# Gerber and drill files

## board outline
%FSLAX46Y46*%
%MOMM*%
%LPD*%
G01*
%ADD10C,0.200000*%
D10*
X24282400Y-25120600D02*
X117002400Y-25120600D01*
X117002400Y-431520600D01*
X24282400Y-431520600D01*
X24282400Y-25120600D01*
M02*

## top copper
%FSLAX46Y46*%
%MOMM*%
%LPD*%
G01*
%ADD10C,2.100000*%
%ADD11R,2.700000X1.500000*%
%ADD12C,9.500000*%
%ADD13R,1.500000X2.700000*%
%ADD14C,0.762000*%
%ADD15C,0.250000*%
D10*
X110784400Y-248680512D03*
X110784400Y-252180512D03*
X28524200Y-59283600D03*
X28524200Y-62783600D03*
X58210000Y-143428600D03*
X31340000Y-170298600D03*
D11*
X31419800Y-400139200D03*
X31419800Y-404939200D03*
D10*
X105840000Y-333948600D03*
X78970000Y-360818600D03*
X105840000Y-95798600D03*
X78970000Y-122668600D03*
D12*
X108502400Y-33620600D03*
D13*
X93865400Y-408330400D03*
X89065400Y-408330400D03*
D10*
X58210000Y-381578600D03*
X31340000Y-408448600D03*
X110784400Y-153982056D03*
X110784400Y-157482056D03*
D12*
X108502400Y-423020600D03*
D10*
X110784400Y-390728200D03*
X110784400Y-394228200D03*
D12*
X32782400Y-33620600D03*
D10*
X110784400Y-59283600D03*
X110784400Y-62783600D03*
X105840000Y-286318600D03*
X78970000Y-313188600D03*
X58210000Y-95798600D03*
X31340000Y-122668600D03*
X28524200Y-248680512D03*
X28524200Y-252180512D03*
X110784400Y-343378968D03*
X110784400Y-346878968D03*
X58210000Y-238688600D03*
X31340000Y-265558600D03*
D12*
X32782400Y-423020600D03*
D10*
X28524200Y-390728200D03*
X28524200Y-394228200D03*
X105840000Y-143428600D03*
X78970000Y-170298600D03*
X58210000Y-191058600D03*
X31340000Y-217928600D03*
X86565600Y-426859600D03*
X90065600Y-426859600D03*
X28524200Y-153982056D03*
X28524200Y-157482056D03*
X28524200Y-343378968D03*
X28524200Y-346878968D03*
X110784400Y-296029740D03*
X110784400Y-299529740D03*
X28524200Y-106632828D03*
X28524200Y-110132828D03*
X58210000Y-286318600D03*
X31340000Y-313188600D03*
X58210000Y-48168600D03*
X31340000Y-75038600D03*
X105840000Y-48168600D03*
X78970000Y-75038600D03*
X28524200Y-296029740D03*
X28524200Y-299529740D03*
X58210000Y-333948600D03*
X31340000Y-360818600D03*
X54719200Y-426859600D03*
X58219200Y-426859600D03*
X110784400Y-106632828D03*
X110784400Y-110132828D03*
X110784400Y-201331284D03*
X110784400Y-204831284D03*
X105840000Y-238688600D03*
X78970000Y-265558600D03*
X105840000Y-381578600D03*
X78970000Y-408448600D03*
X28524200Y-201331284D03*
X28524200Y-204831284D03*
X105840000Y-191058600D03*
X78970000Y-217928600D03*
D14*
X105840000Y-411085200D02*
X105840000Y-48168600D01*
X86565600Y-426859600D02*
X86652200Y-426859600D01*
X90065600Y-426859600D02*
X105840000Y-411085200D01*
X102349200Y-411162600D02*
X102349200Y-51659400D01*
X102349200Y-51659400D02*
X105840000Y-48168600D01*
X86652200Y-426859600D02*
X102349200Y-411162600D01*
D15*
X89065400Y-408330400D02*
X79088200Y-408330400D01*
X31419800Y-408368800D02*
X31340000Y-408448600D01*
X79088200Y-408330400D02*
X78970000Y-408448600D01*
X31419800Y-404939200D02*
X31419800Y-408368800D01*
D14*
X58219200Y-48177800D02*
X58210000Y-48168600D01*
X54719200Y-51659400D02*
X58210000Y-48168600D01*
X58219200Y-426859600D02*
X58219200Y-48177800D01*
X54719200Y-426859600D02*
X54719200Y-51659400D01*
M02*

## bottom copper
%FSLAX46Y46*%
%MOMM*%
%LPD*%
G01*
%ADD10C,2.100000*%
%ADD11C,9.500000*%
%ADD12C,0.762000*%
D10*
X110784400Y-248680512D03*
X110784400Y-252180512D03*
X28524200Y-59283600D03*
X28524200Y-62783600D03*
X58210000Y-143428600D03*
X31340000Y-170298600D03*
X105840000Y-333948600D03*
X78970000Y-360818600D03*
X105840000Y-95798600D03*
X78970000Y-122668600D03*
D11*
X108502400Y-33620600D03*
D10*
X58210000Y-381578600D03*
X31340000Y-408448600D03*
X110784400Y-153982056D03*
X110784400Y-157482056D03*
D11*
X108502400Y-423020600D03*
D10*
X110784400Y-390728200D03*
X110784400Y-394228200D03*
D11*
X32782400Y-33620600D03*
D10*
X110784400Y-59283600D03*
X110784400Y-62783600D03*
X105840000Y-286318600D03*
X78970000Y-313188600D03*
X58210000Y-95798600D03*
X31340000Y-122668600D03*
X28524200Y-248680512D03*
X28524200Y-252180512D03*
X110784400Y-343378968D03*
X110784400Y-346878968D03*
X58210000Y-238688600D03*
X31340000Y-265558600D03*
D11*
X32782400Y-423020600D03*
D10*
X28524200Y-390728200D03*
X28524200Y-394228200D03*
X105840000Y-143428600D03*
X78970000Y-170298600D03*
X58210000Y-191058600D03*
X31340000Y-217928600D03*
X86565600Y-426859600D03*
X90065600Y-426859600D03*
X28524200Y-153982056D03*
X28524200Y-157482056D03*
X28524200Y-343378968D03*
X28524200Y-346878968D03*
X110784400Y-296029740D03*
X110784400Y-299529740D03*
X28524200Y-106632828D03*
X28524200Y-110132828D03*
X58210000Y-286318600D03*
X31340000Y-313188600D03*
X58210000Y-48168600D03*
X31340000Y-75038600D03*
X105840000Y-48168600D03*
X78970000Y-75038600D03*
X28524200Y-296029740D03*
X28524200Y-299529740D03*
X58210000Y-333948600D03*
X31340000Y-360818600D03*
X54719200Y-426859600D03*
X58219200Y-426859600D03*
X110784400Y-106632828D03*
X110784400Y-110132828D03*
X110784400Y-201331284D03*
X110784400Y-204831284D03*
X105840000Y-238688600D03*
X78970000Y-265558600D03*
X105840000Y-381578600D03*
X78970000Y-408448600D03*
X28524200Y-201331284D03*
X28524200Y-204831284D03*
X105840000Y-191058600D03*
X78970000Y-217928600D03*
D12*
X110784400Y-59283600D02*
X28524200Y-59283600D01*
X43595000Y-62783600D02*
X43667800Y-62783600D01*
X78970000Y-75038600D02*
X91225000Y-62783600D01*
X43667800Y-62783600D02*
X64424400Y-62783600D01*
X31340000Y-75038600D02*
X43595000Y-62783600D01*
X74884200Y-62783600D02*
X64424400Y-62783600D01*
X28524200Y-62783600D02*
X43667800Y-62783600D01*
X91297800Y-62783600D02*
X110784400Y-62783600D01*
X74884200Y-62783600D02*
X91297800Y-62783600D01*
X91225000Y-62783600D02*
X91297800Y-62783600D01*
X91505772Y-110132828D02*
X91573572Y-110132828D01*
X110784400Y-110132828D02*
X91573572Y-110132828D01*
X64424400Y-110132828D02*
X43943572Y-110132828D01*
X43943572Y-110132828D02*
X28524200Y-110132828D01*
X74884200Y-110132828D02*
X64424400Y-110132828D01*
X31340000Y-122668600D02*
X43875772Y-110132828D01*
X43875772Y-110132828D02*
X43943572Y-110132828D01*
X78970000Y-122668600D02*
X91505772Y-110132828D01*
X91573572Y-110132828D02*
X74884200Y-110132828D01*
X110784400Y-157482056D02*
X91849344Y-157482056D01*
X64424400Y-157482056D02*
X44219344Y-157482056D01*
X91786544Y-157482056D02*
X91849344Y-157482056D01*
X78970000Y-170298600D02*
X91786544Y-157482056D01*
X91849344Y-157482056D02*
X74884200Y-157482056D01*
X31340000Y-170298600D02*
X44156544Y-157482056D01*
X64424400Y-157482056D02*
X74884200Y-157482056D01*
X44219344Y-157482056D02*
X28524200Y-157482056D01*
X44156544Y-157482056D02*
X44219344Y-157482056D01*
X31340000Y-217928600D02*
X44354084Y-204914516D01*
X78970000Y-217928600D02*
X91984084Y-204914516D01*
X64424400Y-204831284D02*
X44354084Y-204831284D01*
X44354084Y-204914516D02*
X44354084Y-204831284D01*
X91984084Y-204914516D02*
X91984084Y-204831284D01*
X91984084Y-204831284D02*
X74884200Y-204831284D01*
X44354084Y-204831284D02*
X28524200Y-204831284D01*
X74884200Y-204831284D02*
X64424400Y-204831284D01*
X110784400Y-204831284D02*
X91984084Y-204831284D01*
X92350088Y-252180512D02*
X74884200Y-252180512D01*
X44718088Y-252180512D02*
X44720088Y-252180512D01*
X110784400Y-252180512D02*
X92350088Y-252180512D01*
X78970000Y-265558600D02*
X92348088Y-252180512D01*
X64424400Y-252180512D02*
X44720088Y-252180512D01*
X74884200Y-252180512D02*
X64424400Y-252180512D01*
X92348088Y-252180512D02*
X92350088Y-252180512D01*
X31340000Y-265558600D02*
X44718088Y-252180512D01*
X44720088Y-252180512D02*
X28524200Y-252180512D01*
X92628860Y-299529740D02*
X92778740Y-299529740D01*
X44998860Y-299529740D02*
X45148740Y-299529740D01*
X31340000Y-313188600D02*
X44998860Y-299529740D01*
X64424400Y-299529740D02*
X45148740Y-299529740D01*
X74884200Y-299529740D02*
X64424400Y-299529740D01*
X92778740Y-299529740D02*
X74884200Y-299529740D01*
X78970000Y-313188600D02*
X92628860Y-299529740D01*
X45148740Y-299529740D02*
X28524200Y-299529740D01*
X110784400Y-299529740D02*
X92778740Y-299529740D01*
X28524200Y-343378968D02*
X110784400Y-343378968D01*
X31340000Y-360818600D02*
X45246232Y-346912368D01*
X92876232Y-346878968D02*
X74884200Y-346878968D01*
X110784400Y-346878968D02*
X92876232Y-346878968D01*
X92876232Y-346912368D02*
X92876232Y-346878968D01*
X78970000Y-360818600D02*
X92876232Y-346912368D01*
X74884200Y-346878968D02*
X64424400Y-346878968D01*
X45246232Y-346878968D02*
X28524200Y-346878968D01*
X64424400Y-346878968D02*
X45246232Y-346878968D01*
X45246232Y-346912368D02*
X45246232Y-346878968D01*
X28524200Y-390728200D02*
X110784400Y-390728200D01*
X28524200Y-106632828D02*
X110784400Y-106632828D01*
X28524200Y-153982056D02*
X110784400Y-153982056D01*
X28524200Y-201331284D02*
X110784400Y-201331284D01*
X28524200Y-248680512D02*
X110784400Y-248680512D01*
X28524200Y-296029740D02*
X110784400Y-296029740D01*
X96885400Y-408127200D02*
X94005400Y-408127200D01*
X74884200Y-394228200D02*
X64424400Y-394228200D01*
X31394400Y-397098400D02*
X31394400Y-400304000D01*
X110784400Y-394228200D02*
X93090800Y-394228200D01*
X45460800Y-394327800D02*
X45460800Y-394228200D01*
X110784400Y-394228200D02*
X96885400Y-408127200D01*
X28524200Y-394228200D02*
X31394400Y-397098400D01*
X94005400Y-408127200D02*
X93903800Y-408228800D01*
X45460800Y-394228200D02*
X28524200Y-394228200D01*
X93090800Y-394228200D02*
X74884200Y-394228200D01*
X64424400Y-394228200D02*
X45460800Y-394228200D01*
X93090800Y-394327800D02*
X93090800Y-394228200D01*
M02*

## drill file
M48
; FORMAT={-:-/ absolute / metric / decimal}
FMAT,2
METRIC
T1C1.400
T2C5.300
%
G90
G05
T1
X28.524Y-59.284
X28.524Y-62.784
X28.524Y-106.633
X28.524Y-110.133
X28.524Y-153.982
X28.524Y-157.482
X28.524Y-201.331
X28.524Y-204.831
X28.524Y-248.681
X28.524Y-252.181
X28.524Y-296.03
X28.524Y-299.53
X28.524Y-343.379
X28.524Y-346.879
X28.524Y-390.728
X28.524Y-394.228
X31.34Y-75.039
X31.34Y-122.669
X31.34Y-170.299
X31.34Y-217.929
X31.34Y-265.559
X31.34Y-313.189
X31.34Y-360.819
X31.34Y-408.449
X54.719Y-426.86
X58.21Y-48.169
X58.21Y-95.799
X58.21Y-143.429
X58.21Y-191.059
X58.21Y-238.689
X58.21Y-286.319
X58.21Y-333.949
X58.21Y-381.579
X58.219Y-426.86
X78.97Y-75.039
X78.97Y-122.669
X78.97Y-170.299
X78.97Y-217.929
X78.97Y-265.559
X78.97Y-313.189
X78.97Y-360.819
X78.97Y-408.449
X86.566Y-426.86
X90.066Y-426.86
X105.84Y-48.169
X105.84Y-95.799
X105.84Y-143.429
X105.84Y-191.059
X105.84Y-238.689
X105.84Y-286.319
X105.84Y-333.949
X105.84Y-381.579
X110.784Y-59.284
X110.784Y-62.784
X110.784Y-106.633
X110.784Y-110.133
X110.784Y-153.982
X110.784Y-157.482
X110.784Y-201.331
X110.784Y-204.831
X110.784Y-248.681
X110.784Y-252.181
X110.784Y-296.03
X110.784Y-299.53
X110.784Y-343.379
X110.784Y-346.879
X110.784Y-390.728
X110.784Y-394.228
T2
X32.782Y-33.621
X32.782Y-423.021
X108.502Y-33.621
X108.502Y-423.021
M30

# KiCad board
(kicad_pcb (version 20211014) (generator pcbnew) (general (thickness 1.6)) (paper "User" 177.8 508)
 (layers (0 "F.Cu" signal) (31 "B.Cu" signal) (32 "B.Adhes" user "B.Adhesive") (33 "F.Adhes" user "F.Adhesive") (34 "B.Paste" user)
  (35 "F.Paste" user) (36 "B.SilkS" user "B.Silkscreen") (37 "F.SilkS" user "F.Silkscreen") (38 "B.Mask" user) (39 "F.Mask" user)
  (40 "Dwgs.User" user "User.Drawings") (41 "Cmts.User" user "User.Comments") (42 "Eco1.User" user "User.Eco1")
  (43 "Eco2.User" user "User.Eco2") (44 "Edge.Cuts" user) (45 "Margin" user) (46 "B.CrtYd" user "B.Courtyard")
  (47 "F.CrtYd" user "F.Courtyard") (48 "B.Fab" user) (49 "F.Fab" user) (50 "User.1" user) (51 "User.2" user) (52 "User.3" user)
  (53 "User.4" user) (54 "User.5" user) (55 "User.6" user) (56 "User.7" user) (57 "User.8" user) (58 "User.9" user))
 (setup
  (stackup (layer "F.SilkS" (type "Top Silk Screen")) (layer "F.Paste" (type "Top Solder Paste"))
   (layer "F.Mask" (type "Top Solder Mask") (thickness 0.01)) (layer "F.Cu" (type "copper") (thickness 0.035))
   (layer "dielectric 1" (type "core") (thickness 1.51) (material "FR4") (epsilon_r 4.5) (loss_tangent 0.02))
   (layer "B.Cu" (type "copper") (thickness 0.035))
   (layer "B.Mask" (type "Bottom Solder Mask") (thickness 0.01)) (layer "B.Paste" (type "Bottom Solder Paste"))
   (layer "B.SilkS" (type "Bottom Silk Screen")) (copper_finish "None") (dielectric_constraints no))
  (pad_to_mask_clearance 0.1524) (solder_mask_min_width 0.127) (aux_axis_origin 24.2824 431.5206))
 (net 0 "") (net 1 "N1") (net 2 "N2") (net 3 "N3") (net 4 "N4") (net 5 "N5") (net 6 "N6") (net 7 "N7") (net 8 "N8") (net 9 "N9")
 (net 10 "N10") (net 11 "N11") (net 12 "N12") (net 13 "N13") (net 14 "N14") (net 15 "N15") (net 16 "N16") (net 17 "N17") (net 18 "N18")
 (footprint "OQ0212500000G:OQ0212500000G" (layer "F.Cu") (at 110.7844 248.680512 -90)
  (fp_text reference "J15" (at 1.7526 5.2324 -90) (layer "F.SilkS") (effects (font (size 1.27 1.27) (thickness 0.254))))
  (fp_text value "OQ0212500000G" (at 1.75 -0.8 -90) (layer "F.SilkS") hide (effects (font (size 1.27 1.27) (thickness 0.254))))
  (pad "1" thru_hole circle (at 0 0 270) (size 2.1 2.1) (drill 1.4) (layers F&B.Cu *.Mask) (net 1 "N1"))
  (pad "2" thru_hole circle (at 3.5 0 270) (size 2.1 2.1) (drill 1.4) (layers F&B.Cu *.Mask) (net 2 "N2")))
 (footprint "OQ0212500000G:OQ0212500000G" (layer "F.Cu") (at 28.5242 59.2836 -90)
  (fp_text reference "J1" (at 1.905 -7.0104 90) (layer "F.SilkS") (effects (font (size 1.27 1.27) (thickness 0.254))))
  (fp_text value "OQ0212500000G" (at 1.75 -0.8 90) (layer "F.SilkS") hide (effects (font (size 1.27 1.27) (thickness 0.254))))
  (pad "1" thru_hole circle (at 0 0 270) (size 2.1 2.1) (drill 1.4) (layers *.Cu *.Mask) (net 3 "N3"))
  (pad "2" thru_hole circle (at 3.5 0 270) (size 2.1 2.1) (drill 1.4) (layers *.Cu *.Mask) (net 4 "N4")))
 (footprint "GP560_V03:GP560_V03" (layer "F.Cu") (at 31.34 170.2986)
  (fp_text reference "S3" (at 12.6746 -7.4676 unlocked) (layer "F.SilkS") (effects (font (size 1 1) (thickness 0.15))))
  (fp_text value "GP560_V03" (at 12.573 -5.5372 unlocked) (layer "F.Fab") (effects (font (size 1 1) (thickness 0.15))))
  (pad "1" thru_hole circle (at 26.87 -26.87) (size 2.1 2.1) (drill 1.4) (layers *.Cu *.Mask) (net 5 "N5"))
  (pad "2" thru_hole circle (at 0 0) (size 2.1 2.1) (drill 1.4) (layers *.Cu *.Mask) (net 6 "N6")))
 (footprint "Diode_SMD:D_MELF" (layer "F.Cu") (at 31.4198 402.5392 -90)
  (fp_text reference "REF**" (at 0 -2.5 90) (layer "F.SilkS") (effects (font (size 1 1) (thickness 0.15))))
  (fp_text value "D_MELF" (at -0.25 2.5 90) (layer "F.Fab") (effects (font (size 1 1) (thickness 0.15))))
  (pad "1" smd rect (at -2.4 0 270) (size 1.5 2.7) (layers "F.Cu" "F.Paste" "F.Mask") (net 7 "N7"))
  (pad "2" smd rect (at 2.4 0 270) (size 1.5 2.7) (layers "F.Cu" "F.Paste" "F.Mask") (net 7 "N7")))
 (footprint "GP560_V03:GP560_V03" (layer "F.Cu") (at 78.97 360.8186)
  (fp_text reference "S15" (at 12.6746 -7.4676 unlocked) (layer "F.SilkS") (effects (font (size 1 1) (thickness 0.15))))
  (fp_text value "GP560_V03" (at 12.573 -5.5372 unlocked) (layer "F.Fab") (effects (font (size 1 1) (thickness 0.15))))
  (pad "1" thru_hole circle (at 26.87 -26.87) (size 2.1 2.1) (drill 1.4) (layers *.Cu *.Mask) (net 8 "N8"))
  (pad "2" thru_hole circle (at 0 0) (size 2.1 2.1) (drill 1.4) (layers *.Cu *.Mask) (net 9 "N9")))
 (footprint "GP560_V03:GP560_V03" (layer "F.Cu") (at 78.97 122.6686)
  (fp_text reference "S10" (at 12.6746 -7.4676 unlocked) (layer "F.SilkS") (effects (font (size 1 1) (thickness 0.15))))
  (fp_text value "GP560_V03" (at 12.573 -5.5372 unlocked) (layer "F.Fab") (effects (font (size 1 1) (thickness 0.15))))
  (pad "1" thru_hole circle (at 26.87 -26.87) (size 2.1 2.1) (drill 1.4) (layers *.Cu *.Mask) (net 8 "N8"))
  (pad "2" thru_hole circle (at 0 0) (size 2.1 2.1) (drill 1.4) (layers *.Cu *.Mask) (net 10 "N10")))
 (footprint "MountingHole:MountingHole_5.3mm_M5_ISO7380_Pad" (layer "F.Cu") (at 108.5024 33.6206)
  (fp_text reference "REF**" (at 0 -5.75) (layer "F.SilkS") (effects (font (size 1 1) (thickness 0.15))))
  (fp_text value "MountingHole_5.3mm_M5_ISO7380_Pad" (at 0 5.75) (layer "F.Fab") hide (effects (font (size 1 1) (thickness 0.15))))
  (pad "1" thru_hole circle (at 0 0) (size 9.5 9.5) (drill 5.3) (layers F&B.Cu *.Mask)))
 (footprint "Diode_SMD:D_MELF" (layer "F.Cu") (at 91.4654 408.3304 180)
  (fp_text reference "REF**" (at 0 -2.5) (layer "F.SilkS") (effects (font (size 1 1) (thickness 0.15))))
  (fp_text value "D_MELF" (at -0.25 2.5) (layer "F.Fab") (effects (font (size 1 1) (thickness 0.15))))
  (pad "1" smd rect (at -2.4 0 180) (size 1.5 2.7) (layers "F.Cu" "F.Paste" "F.Mask") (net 7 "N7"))
  (pad "2" smd rect (at 2.4 0 180) (size 1.5 2.7) (layers "F.Cu" "F.Paste" "F.Mask") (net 7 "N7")))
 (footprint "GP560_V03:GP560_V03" (layer "F.Cu") (at 31.34 408.4486)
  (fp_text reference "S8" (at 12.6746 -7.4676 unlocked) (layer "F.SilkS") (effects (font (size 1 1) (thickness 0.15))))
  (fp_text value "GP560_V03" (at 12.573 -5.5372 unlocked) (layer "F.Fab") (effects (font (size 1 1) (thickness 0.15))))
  (pad "1" thru_hole circle (at 26.87 -26.87) (size 2.1 2.1) (drill 1.4) (layers *.Cu *.Mask) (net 5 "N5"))
  (pad "2" thru_hole circle (at 0 0) (size 2.1 2.1) (drill 1.4) (layers *.Cu *.Mask) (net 7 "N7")))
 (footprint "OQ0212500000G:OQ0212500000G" (layer "F.Cu") (at 110.7844 153.982056 -90)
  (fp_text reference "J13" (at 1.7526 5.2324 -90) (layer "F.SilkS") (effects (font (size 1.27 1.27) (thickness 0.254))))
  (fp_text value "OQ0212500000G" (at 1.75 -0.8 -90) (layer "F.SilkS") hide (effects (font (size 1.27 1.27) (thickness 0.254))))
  (pad "1" thru_hole circle (at 0 0 270) (size 2.1 2.1) (drill 1.4) (layers F&B.Cu *.Mask) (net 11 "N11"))
  (pad "2" thru_hole circle (at 3.5 0 270) (size 2.1 2.1) (drill 1.4) (layers F&B.Cu *.Mask) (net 6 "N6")))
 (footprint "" (layer "F.Cu") (at 108.5024 423.0206)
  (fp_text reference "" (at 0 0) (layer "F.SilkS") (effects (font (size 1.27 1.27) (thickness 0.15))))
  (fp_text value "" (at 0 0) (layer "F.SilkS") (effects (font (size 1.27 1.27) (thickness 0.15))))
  (pad "1" thru_hole circle (at 0 0) (size 9.5 9.5) (drill 5.3) (layers F&B.Cu *.Mask)))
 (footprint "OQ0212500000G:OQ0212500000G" (layer "F.Cu") (at 110.7844 390.7282 -90)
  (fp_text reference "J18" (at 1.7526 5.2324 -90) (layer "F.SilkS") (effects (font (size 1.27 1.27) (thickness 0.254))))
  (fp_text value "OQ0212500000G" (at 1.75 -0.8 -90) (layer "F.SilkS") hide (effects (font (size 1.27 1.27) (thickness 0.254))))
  (pad "1" thru_hole circle (at 0 0 270) (size 2.1 2.1) (drill 1.4) (layers F&B.Cu *.Mask) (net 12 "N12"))
  (pad "2" thru_hole circle (at 3.5 0 270) (size 2.1 2.1) (drill 1.4) (layers F&B.Cu *.Mask) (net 7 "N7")))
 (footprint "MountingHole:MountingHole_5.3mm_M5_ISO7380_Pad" (layer "F.Cu") (at 32.7824 33.6206)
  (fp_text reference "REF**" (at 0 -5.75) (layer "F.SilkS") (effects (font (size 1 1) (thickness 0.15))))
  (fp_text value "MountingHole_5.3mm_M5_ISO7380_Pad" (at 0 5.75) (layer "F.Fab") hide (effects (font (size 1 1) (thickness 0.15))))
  (pad "1" thru_hole circle (at 0 0) (size 9.5 9.5) (drill 5.3) (layers F&B.Cu *.Mask)))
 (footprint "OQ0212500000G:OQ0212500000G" (layer "F.Cu") (at 110.7844 59.2836 -90)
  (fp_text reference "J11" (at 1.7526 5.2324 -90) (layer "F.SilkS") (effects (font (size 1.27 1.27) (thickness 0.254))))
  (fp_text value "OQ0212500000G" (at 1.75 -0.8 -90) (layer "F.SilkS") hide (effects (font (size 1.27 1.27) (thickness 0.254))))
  (pad "1" thru_hole circle (at 0 0 270) (size 2.1 2.1) (drill 1.4) (layers F&B.Cu *.Mask) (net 3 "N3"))
  (pad "2" thru_hole circle (at 3.5 0 270) (size 2.1 2.1) (drill 1.4) (layers F&B.Cu *.Mask) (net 4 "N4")))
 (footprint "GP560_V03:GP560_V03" (layer "F.Cu") (at 78.97 313.1886)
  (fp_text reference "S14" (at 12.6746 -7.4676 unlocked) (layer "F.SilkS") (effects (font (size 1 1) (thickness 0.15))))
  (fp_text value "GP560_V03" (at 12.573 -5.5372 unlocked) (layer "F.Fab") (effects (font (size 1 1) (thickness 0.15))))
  (pad "1" thru_hole circle (at 26.87 -26.87) (size 2.1 2.1) (drill 1.4) (layers *.Cu *.Mask) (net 8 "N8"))
  (pad "2" thru_hole circle (at 0 0) (size 2.1 2.1) (drill 1.4) (layers *.Cu *.Mask) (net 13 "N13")))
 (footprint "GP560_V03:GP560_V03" (layer "F.Cu") (at 31.34 122.6686)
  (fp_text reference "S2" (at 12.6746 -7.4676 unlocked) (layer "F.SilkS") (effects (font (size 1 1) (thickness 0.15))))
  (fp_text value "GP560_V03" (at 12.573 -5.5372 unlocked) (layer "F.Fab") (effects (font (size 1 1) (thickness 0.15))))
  (pad "1" thru_hole circle (at 26.87 -26.87) (size 2.1 2.1) (drill 1.4) (layers *.Cu *.Mask) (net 5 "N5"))
  (pad "2" thru_hole circle (at 0 0) (size 2.1 2.1) (drill 1.4) (layers *.Cu *.Mask) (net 10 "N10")))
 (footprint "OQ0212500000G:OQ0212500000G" (layer "F.Cu") (at 28.5242 248.680512 -90)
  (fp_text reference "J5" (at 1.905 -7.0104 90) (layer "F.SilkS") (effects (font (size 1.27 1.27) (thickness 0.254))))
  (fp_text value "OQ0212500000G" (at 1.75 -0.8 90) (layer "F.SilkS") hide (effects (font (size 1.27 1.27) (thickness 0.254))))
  (pad "1" thru_hole circle (at 0 0 270) (size 2.1 2.1) (drill 1.4) (layers *.Cu *.Mask) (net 1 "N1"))
  (pad "2" thru_hole circle (at 3.5 0 270) (size 2.1 2.1) (drill 1.4) (layers *.Cu *.Mask) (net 2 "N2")))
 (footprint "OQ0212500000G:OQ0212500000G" (layer "F.Cu") (at 110.7844 343.378968 -90)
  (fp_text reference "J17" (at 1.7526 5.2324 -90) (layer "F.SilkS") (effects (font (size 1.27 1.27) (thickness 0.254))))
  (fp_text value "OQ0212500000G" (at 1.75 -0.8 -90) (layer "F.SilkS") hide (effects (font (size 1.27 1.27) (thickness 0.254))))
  (pad "1" thru_hole circle (at 0 0 270) (size 2.1 2.1) (drill 1.4) (layers F&B.Cu *.Mask) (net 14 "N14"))
  (pad "2" thru_hole circle (at 3.5 0 270) (size 2.1 2.1) (drill 1.4) (layers F&B.Cu *.Mask) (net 9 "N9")))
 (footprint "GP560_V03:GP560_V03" (layer "F.Cu") (at 31.34 265.5586)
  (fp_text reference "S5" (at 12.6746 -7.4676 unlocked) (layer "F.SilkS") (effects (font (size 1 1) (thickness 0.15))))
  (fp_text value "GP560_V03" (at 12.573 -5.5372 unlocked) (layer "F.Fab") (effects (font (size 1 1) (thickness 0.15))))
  (pad "1" thru_hole circle (at 26.87 -26.87) (size 2.1 2.1) (drill 1.4) (layers *.Cu *.Mask) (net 5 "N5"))
  (pad "2" thru_hole circle (at 0 0) (size 2.1 2.1) (drill 1.4) (layers *.Cu *.Mask) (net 2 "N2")))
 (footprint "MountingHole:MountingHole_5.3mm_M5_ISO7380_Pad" (layer "F.Cu") (at 32.7824 423.0206)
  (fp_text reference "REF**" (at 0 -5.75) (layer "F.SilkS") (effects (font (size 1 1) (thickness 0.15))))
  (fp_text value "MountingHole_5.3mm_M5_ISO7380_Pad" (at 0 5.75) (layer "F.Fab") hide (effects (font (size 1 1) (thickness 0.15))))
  (pad "1" thru_hole circle (at 0 0) (size 9.5 9.5) (drill 5.3) (layers *.Cu *.Mask)))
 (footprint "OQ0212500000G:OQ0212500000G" (layer "F.Cu") (at 28.5242 390.7282 -90)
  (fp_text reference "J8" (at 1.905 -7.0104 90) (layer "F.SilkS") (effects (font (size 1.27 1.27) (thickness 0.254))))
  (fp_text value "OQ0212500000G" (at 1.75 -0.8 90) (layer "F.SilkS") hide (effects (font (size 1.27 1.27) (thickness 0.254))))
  (pad "1" thru_hole circle (at 0 0 270) (size 2.1 2.1) (drill 1.4) (layers *.Cu *.Mask) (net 12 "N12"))
  (pad "2" thru_hole circle (at 3.5 0 270) (size 2.1 2.1) (drill 1.4) (layers *.Cu *.Mask) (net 7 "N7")))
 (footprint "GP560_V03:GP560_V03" (layer "F.Cu") (at 78.97 170.2986)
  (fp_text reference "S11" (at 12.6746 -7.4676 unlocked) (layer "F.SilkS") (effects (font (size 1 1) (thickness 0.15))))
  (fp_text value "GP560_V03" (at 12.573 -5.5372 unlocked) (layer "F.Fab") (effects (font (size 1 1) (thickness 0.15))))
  (pad "1" thru_hole circle (at 26.87 -26.87) (size 2.1 2.1) (drill 1.4) (layers *.Cu *.Mask) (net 8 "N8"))
  (pad "2" thru_hole circle (at 0 0) (size 2.1 2.1) (drill 1.4) (layers *.Cu *.Mask) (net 6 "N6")))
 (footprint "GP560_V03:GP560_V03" (layer "F.Cu") (at 31.34 217.9286)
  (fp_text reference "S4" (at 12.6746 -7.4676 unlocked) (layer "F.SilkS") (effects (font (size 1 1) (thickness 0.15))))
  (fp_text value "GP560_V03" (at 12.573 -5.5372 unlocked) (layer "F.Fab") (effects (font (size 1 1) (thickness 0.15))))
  (pad "1" thru_hole circle (at 26.87 -26.87) (size 2.1 2.1) (drill 1.4) (layers *.Cu *.Mask) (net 5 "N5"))
  (pad "2" thru_hole circle (at 0 0) (size 2.1 2.1) (drill 1.4) (layers *.Cu *.Mask) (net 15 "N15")))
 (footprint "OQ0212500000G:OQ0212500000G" (layer "F.Cu") (at 86.5656 426.8596)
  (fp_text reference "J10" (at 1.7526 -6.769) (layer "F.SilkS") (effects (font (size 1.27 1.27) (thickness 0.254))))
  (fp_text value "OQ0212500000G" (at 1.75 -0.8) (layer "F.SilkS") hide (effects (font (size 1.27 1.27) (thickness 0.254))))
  (pad "1" thru_hole circle (at 0 0) (size 2.1 2.1) (drill 1.4) (layers *.Cu *.Mask) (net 8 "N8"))
  (pad "2" thru_hole circle (at 3.5 0) (size 2.1 2.1) (drill 1.4) (layers *.Cu *.Mask) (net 8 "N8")))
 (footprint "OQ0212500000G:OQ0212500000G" (layer "F.Cu") (at 28.5242 153.982056 -90)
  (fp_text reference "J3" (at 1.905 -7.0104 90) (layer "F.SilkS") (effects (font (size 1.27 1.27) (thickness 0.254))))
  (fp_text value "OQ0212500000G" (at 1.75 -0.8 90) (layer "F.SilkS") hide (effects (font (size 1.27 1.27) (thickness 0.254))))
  (pad "1" thru_hole circle (at 0 0 270) (size 2.1 2.1) (drill 1.4) (layers *.Cu *.Mask) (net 11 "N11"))
  (pad "2" thru_hole circle (at 3.5 0 270) (size 2.1 2.1) (drill 1.4) (layers *.Cu *.Mask) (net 6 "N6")))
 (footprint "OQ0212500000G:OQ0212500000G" (layer "F.Cu") (at 28.5242 343.378968 -90)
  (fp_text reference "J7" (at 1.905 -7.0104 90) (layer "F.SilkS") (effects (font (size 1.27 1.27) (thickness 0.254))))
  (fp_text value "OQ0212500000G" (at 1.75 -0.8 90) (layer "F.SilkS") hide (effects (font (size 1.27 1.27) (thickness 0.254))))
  (pad "1" thru_hole circle (at 0 0 270) (size 2.1 2.1) (drill 1.4) (layers *.Cu *.Mask) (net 14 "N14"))
  (pad "2" thru_hole circle (at 3.5 0 270) (size 2.1 2.1) (drill 1.4) (layers *.Cu *.Mask) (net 9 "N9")))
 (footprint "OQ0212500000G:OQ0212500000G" (layer "F.Cu") (at 110.7844 296.02974 -90)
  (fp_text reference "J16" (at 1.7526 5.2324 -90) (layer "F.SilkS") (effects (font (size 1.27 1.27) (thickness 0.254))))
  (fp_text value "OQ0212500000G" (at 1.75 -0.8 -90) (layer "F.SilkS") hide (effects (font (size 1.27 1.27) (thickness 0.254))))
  (pad "1" thru_hole circle (at 0 0 270) (size 2.1 2.1) (drill 1.4) (layers F&B.Cu *.Mask) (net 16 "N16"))
  (pad "2" thru_hole circle (at 3.5 0 270) (size 2.1 2.1) (drill 1.4) (layers F&B.Cu *.Mask) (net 13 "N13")))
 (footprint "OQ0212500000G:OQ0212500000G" (layer "F.Cu") (at 28.5242 106.632828 -90)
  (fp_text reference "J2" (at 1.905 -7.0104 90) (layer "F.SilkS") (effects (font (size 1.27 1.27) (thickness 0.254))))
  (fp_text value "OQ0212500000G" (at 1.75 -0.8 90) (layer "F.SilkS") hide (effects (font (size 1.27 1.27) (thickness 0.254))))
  (pad "1" thru_hole circle (at 0 0 270) (size 2.1 2.1) (drill 1.4) (layers *.Cu *.Mask) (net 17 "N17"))
  (pad "2" thru_hole circle (at 3.5 0 270) (size 2.1 2.1) (drill 1.4) (layers *.Cu *.Mask) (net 10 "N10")))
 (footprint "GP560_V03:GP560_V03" (layer "F.Cu") (at 31.34 313.1886)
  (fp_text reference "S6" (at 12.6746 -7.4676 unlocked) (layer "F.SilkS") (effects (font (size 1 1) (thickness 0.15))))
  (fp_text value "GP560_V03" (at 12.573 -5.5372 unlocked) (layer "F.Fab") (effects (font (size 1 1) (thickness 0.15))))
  (pad "1" thru_hole circle (at 26.87 -26.87) (size 2.1 2.1) (drill 1.4) (layers *.Cu *.Mask) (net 5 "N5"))
  (pad "2" thru_hole circle (at 0 0) (size 2.1 2.1) (drill 1.4) (layers *.Cu *.Mask) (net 13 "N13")))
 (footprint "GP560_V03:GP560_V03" (layer "F.Cu") (at 31.34 75.0386)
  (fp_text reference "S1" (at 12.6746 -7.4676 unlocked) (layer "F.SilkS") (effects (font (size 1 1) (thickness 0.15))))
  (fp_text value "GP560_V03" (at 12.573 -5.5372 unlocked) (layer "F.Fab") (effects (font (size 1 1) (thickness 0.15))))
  (pad "1" thru_hole circle (at 26.87 -26.87) (size 2.1 2.1) (drill 1.4) (layers *.Cu *.Mask) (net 5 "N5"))
  (pad "2" thru_hole circle (at 0 0) (size 2.1 2.1) (drill 1.4) (layers *.Cu *.Mask) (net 4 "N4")))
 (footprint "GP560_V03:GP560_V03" (layer "F.Cu") (at 78.97 75.0386)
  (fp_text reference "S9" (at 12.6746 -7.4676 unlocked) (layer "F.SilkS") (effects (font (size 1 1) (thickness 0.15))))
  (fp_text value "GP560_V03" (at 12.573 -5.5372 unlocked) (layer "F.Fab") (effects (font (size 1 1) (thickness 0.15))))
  (pad "1" thru_hole circle (at 26.87 -26.87) (size 2.1 2.1) (drill 1.4) (layers *.Cu *.Mask) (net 8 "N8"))
  (pad "2" thru_hole circle (at 0 0) (size 2.1 2.1) (drill 1.4) (layers *.Cu *.Mask) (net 4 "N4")))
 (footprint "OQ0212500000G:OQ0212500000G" (layer "F.Cu") (at 28.5242 296.02974 -90)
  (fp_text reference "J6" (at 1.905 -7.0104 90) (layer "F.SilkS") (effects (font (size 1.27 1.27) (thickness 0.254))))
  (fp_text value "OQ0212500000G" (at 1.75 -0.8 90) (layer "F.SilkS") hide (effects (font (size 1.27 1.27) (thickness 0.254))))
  (pad "1" thru_hole circle (at 0 0 270) (size 2.1 2.1) (drill 1.4) (layers *.Cu *.Mask) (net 16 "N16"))
  (pad "2" thru_hole circle (at 3.5 0 270) (size 2.1 2.1) (drill 1.4) (layers *.Cu *.Mask) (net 13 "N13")))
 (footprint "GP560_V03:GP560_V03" (layer "F.Cu") (at 31.34 360.8186)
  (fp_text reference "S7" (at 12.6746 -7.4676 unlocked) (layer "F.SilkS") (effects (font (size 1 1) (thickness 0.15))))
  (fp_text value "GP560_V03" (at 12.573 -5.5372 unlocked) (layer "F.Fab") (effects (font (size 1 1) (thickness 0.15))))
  (pad "1" thru_hole circle (at 26.87 -26.87) (size 2.1 2.1) (drill 1.4) (layers *.Cu *.Mask) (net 5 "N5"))
  (pad "2" thru_hole circle (at 0 0) (size 2.1 2.1) (drill 1.4) (layers *.Cu *.Mask) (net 9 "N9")))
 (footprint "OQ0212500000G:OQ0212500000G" (layer "F.Cu") (at 54.7192 426.8596)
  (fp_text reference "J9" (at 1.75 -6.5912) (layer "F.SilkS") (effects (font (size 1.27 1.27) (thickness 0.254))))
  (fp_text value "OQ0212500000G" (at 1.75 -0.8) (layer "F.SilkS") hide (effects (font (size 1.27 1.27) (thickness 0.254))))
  (pad "1" thru_hole circle (at 0 0) (size 2.1 2.1) (drill 1.4) (layers *.Cu *.Mask) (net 5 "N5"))
  (pad "2" thru_hole circle (at 3.5 0) (size 2.1 2.1) (drill 1.4) (layers *.Cu *.Mask) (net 5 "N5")))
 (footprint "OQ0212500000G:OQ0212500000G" (layer "F.Cu") (at 110.7844 106.632828 -90)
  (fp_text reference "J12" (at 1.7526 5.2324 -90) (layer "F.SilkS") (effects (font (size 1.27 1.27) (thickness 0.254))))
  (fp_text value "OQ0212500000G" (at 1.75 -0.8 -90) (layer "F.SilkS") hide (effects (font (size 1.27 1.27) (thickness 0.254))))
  (pad "1" thru_hole circle (at 0 0 270) (size 2.1 2.1) (drill 1.4) (layers F&B.Cu *.Mask) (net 17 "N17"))
  (pad "2" thru_hole circle (at 3.5 0 270) (size 2.1 2.1) (drill 1.4) (layers F&B.Cu *.Mask) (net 10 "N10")))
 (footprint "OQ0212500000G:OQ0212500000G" (layer "F.Cu") (at 110.7844 201.331284 -90)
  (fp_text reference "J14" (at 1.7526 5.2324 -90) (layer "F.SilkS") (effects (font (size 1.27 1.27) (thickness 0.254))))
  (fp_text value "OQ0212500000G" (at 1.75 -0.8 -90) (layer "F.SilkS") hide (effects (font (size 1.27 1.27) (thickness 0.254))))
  (pad "1" thru_hole circle (at 0 0 270) (size 2.1 2.1) (drill 1.4) (layers F&B.Cu *.Mask) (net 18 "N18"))
  (pad "2" thru_hole circle (at 3.5 0 270) (size 2.1 2.1) (drill 1.4) (layers F&B.Cu *.Mask) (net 15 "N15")))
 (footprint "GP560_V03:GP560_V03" (layer "F.Cu") (at 78.97 265.5586)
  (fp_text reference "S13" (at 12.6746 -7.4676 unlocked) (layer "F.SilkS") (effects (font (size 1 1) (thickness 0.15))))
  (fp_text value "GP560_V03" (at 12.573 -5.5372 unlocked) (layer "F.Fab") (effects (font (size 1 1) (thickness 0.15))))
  (pad "1" thru_hole circle (at 26.87 -26.87) (size 2.1 2.1) (drill 1.4) (layers *.Cu *.Mask) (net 8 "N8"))
  (pad "2" thru_hole circle (at 0 0) (size 2.1 2.1) (drill 1.4) (layers *.Cu *.Mask) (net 2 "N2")))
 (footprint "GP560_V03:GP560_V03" (layer "F.Cu") (at 78.97 408.4486)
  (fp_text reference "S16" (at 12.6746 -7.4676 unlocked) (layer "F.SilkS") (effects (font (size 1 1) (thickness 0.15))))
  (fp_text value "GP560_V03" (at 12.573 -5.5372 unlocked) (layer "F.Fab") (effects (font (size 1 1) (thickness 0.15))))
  (pad "1" thru_hole circle (at 26.87 -26.87) (size 2.1 2.1) (drill 1.4) (layers *.Cu *.Mask) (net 8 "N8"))
  (pad "2" thru_hole circle (at 0 0) (size 2.1 2.1) (drill 1.4) (layers *.Cu *.Mask) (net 7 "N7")))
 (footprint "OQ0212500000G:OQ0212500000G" (layer "F.Cu") (at 28.5242 201.331284 -90)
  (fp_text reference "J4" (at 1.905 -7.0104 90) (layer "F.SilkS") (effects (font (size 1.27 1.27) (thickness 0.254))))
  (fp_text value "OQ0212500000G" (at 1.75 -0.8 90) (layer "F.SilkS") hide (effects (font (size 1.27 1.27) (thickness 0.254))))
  (pad "1" thru_hole circle (at 0 0 270) (size 2.1 2.1) (drill 1.4) (layers *.Cu *.Mask) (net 18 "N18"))
  (pad "2" thru_hole circle (at 3.5 0 270) (size 2.1 2.1) (drill 1.4) (layers *.Cu *.Mask) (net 15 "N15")))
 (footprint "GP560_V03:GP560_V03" (layer "F.Cu") (at 78.97 217.9286)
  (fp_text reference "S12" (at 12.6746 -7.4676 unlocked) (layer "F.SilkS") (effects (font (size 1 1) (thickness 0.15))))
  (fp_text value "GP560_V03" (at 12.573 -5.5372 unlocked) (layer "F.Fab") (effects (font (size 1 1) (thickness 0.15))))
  (pad "1" thru_hole circle (at 26.87 -26.87) (size 2.1 2.1) (drill 1.4) (layers *.Cu *.Mask) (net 8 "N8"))
  (pad "2" thru_hole circle (at 0 0) (size 2.1 2.1) (drill 1.4) (layers *.Cu *.Mask) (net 15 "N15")))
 (gr_rect (start 24.2824 431.5206) (end 117.0024 25.1206) (layer "Edge.Cuts") (width 0.2) (fill none))
 (segment (start 110.7844 59.2836) (end 28.5242 59.2836) (width 0.762) (layer "B.Cu") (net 3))
 (segment (start 43.595 62.7836) (end 43.6678 62.7836) (width 0.762) (layer "B.Cu") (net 4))
 (segment (start 78.97 75.0386) (end 91.225 62.7836) (width 0.762) (layer "B.Cu") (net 4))
 (segment (start 43.6678 62.7836) (end 64.4244 62.7836) (width 0.762) (layer "B.Cu") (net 4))
 (segment (start 31.34 75.0386) (end 43.595 62.7836) (width 0.762) (layer "B.Cu") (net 4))
 (segment (start 74.8842 62.7836) (end 64.4244 62.7836) (width 0.762) (layer "B.Cu") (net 4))
 (segment (start 28.5242 62.7836) (end 43.6678 62.7836) (width 0.762) (layer "B.Cu") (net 4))
 (segment (start 91.2978 62.7836) (end 110.7844 62.7836) (width 0.762) (layer "B.Cu") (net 4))
 (segment (start 74.8842 62.7836) (end 91.2978 62.7836) (width 0.762) (layer "B.Cu") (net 4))
 (segment (start 91.225 62.7836) (end 91.2978 62.7836) (width 0.762) (layer "B.Cu") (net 4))
 (segment (start 91.505772 110.132828) (end 91.573572 110.132828) (width 0.762) (layer "B.Cu") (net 10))
 (segment (start 110.7844 110.132828) (end 91.573572 110.132828) (width 0.762) (layer "B.Cu") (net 10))
 (segment (start 64.4244 110.132828) (end 43.943572 110.132828) (width 0.762) (layer "B.Cu") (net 10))
 (segment (start 43.943572 110.132828) (end 28.5242 110.132828) (width 0.762) (layer "B.Cu") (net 10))
 (segment (start 74.8842 110.132828) (end 64.4244 110.132828) (width 0.762) (layer "B.Cu") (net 10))
 (segment (start 31.34 122.6686) (end 43.875772 110.132828) (width 0.762) (layer "B.Cu") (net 10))
 (segment (start 43.875772 110.132828) (end 43.943572 110.132828) (width 0.762) (layer "B.Cu") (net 10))
 (segment (start 78.97 122.6686) (end 91.505772 110.132828) (width 0.762) (layer "B.Cu") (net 10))
 (segment (start 91.573572 110.132828) (end 74.8842 110.132828) (width 0.762) (layer "B.Cu") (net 10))
 (segment (start 110.7844 157.482056) (end 91.849344 157.482056) (width 0.762) (layer "B.Cu") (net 6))
 (segment (start 64.4244 157.482056) (end 44.219344 157.482056) (width 0.762) (layer "B.Cu") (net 6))
 (segment (start 91.786544 157.482056) (end 91.849344 157.482056) (width 0.762) (layer "B.Cu") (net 6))
 (segment (start 78.97 170.2986) (end 91.786544 157.482056) (width 0.762) (layer "B.Cu") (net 6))
 (segment (start 91.849344 157.482056) (end 74.8842 157.482056) (width 0.762) (layer "B.Cu") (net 6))
 (segment (start 31.34 170.2986) (end 44.156544 157.482056) (width 0.762) (layer "B.Cu") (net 6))
 (segment (start 64.4244 157.482056) (end 74.8842 157.482056) (width 0.762) (layer "B.Cu") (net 6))
 (segment (start 44.219344 157.482056) (end 28.5242 157.482056) (width 0.762) (layer "B.Cu") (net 6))
 (segment (start 44.156544 157.482056) (end 44.219344 157.482056) (width 0.762) (layer "B.Cu") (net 6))
 (segment (start 31.34 217.9286) (end 44.354084 204.914516) (width 0.762) (layer "B.Cu") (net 15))
 (segment (start 78.97 217.9286) (end 91.984084 204.914516) (width 0.762) (layer "B.Cu") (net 15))
 (segment (start 64.4244 204.831284) (end 44.354084 204.831284) (width 0.762) (layer "B.Cu") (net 15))
 (segment (start 44.354084 204.914516) (end 44.354084 204.831284) (width 0.762) (layer "B.Cu") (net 15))
 (segment (start 91.984084 204.914516) (end 91.984084 204.831284) (width 0.762) (layer "B.Cu") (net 15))
 (segment (start 91.984084 204.831284) (end 74.8842 204.831284) (width 0.762) (layer "B.Cu") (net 15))
 (segment (start 44.354084 204.831284) (end 28.5242 204.831284) (width 0.762) (layer "B.Cu") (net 15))
 (segment (start 74.8842 204.831284) (end 64.4244 204.831284) (width 0.762) (layer "B.Cu") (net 15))
 (segment (start 110.7844 204.831284) (end 91.984084 204.831284) (width 0.762) (layer "B.Cu") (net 15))
 (segment (start 92.350088 252.180512) (end 74.8842 252.180512) (width 0.762) (layer "B.Cu") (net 2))
 (segment (start 44.718088 252.180512) (end 44.720088 252.180512) (width 0.762) (layer "B.Cu") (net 2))
 (segment (start 110.7844 252.180512) (end 92.350088 252.180512) (width 0.762) (layer "B.Cu") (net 2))
 (segment (start 78.97 265.5586) (end 92.348088 252.180512) (width 0.762) (layer "B.Cu") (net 2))
 (segment (start 64.4244 252.180512) (end 44.720088 252.180512) (width 0.762) (layer "B.Cu") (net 2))
 (segment (start 74.8842 252.180512) (end 64.4244 252.180512) (width 0.762) (layer "B.Cu") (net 2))
 (segment (start 92.348088 252.180512) (end 92.350088 252.180512) (width 0.762) (layer "B.Cu") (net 2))
 (segment (start 31.34 265.5586) (end 44.718088 252.180512) (width 0.762) (layer "B.Cu") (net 2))
 (segment (start 44.720088 252.180512) (end 28.5242 252.180512) (width 0.762) (layer "B.Cu") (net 2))
 (segment (start 92.62886 299.52974) (end 92.77874 299.52974) (width 0.762) (layer "B.Cu") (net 13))
 (segment (start 44.99886 299.52974) (end 45.14874 299.52974) (width 0.762) (layer "B.Cu") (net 13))
 (segment (start 31.34 313.1886) (end 44.99886 299.52974) (width 0.762) (layer "B.Cu") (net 13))
 (segment (start 64.4244 299.52974) (end 45.14874 299.52974) (width 0.762) (layer "B.Cu") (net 13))
 (segment (start 74.8842 299.52974) (end 64.4244 299.52974) (width 0.762) (layer "B.Cu") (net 13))
 (segment (start 92.77874 299.52974) (end 74.8842 299.52974) (width 0.762) (layer "B.Cu") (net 13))
 (segment (start 78.97 313.1886) (end 92.62886 299.52974) (width 0.762) (layer "B.Cu") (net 13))
 (segment (start 45.14874 299.52974) (end 28.5242 299.52974) (width 0.762) (layer "B.Cu") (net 13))
 (segment (start 110.7844 299.52974) (end 92.77874 299.52974) (width 0.762) (layer "B.Cu") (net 13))
 (segment (start 28.5242 343.378968) (end 110.7844 343.378968) (width 0.762) (layer "B.Cu") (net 14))
 (segment (start 31.34 360.8186) (end 45.246232 346.912368) (width 0.762) (layer "B.Cu") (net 9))
 (segment (start 92.876232 346.878968) (end 74.8842 346.878968) (width 0.762) (layer "B.Cu") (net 9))
 (segment (start 110.7844 346.878968) (end 92.876232 346.878968) (width 0.762) (layer "B.Cu") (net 9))
 (segment (start 92.876232 346.912368) (end 92.876232 346.878968) (width 0.762) (layer "B.Cu") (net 9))
 (segment (start 78.97 360.8186) (end 92.876232 346.912368) (width 0.762) (layer "B.Cu") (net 9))
 (segment (start 74.8842 346.878968) (end 64.4244 346.878968) (width 0.762) (layer "B.Cu") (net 9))
 (segment (start 45.246232 346.878968) (end 28.5242 346.878968) (width 0.762) (layer "B.Cu") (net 9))
 (segment (start 64.4244 346.878968) (end 45.246232 346.878968) (width 0.762) (layer "B.Cu") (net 9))
 (segment (start 45.246232 346.912368) (end 45.246232 346.878968) (width 0.762) (layer "B.Cu") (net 9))
 (segment (start 105.84 411.0852) (end 105.84 48.1686) (width 0.762) (layer "F.Cu") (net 8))
 (segment (start 86.5656 426.8596) (end 86.6522 426.8596) (width 0.762) (layer "F.Cu") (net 8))
 (segment (start 90.0656 426.8596) (end 105.84 411.0852) (width 0.762) (layer "F.Cu") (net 8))
 (segment (start 102.3492 411.1626) (end 102.3492 51.6594) (width 0.762) (layer "F.Cu") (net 8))
 (segment (start 102.3492 51.6594) (end 105.84 48.1686) (width 0.762) (layer "F.Cu") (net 8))
 (segment (start 86.6522 426.8596) (end 102.3492 411.1626) (width 0.762) (layer "F.Cu") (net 8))
 (segment (start 28.5242 390.7282) (end 110.7844 390.7282) (width 0.762) (layer "B.Cu") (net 12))
 (segment (start 28.5242 106.632828) (end 110.7844 106.632828) (width 0.762) (layer "B.Cu") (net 17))
 (segment (start 28.5242 153.982056) (end 110.7844 153.982056) (width 0.762) (layer "B.Cu") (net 11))
 (segment (start 28.5242 201.331284) (end 110.7844 201.331284) (width 0.762) (layer "B.Cu") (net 18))
 (segment (start 28.5242 248.680512) (end 110.7844 248.680512) (width 0.762) (layer "B.Cu") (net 1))
 (segment (start 28.5242 296.02974) (end 110.7844 296.02974) (width 0.762) (layer "B.Cu") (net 16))
 (segment (start 89.0654 408.3304) (end 79.0882 408.3304) (width 0.25) (layer "F.Cu") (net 7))
 (segment (start 31.4198 408.3688) (end 31.34 408.4486) (width 0.25) (layer "F.Cu") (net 7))
 (segment (start 79.0882 408.3304) (end 78.97 408.4486) (width 0.25) (layer "F.Cu") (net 7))
 (segment (start 31.4198 404.9392) (end 31.4198 408.3688) (width 0.25) (layer "F.Cu") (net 7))
 (segment (start 96.8854 408.1272) (end 94.0054 408.1272) (width 0.762) (layer "B.Cu") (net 7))
 (segment (start 74.8842 394.2282) (end 64.4244 394.2282) (width 0.762) (layer "B.Cu") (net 7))
 (segment (start 31.3944 397.0984) (end 31.3944 400.304) (width 0.762) (layer "B.Cu") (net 7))
 (segment (start 110.7844 394.2282) (end 93.0908 394.2282) (width 0.762) (layer "B.Cu") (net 7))
 (segment (start 45.4608 394.3278) (end 45.4608 394.2282) (width 0.762) (layer "B.Cu") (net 7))
 (segment (start 110.7844 394.2282) (end 96.8854 408.1272) (width 0.762) (layer "B.Cu") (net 7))
 (segment (start 28.5242 394.2282) (end 31.3944 397.0984) (width 0.762) (layer "B.Cu") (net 7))
 (segment (start 94.0054 408.1272) (end 93.9038 408.2288) (width 0.762) (layer "B.Cu") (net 7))
 (segment (start 45.4608 394.2282) (end 28.5242 394.2282) (width 0.762) (layer "B.Cu") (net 7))
 (segment (start 93.0908 394.2282) (end 74.8842 394.2282) (width 0.762) (layer "B.Cu") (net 7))
 (segment (start 64.4244 394.2282) (end 45.4608 394.2282) (width 0.762) (layer "B.Cu") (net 7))
 (segment (start 93.0908 394.3278) (end 93.0908 394.2282) (width 0.762) (layer "B.Cu") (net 7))
 (segment (start 58.2192 48.1778) (end 58.21 48.1686) (width 0.762) (layer "F.Cu") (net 5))
 (segment (start 54.7192 51.6594) (end 58.21 48.1686) (width 0.762) (layer "F.Cu") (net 5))
 (segment (start 58.2192 426.8596) (end 58.2192 48.1778) (width 0.762) (layer "F.Cu") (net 5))
 (segment (start 54.7192 426.8596) (end 54.7192 51.6594) (width 0.762) (layer "F.Cu") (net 5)))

